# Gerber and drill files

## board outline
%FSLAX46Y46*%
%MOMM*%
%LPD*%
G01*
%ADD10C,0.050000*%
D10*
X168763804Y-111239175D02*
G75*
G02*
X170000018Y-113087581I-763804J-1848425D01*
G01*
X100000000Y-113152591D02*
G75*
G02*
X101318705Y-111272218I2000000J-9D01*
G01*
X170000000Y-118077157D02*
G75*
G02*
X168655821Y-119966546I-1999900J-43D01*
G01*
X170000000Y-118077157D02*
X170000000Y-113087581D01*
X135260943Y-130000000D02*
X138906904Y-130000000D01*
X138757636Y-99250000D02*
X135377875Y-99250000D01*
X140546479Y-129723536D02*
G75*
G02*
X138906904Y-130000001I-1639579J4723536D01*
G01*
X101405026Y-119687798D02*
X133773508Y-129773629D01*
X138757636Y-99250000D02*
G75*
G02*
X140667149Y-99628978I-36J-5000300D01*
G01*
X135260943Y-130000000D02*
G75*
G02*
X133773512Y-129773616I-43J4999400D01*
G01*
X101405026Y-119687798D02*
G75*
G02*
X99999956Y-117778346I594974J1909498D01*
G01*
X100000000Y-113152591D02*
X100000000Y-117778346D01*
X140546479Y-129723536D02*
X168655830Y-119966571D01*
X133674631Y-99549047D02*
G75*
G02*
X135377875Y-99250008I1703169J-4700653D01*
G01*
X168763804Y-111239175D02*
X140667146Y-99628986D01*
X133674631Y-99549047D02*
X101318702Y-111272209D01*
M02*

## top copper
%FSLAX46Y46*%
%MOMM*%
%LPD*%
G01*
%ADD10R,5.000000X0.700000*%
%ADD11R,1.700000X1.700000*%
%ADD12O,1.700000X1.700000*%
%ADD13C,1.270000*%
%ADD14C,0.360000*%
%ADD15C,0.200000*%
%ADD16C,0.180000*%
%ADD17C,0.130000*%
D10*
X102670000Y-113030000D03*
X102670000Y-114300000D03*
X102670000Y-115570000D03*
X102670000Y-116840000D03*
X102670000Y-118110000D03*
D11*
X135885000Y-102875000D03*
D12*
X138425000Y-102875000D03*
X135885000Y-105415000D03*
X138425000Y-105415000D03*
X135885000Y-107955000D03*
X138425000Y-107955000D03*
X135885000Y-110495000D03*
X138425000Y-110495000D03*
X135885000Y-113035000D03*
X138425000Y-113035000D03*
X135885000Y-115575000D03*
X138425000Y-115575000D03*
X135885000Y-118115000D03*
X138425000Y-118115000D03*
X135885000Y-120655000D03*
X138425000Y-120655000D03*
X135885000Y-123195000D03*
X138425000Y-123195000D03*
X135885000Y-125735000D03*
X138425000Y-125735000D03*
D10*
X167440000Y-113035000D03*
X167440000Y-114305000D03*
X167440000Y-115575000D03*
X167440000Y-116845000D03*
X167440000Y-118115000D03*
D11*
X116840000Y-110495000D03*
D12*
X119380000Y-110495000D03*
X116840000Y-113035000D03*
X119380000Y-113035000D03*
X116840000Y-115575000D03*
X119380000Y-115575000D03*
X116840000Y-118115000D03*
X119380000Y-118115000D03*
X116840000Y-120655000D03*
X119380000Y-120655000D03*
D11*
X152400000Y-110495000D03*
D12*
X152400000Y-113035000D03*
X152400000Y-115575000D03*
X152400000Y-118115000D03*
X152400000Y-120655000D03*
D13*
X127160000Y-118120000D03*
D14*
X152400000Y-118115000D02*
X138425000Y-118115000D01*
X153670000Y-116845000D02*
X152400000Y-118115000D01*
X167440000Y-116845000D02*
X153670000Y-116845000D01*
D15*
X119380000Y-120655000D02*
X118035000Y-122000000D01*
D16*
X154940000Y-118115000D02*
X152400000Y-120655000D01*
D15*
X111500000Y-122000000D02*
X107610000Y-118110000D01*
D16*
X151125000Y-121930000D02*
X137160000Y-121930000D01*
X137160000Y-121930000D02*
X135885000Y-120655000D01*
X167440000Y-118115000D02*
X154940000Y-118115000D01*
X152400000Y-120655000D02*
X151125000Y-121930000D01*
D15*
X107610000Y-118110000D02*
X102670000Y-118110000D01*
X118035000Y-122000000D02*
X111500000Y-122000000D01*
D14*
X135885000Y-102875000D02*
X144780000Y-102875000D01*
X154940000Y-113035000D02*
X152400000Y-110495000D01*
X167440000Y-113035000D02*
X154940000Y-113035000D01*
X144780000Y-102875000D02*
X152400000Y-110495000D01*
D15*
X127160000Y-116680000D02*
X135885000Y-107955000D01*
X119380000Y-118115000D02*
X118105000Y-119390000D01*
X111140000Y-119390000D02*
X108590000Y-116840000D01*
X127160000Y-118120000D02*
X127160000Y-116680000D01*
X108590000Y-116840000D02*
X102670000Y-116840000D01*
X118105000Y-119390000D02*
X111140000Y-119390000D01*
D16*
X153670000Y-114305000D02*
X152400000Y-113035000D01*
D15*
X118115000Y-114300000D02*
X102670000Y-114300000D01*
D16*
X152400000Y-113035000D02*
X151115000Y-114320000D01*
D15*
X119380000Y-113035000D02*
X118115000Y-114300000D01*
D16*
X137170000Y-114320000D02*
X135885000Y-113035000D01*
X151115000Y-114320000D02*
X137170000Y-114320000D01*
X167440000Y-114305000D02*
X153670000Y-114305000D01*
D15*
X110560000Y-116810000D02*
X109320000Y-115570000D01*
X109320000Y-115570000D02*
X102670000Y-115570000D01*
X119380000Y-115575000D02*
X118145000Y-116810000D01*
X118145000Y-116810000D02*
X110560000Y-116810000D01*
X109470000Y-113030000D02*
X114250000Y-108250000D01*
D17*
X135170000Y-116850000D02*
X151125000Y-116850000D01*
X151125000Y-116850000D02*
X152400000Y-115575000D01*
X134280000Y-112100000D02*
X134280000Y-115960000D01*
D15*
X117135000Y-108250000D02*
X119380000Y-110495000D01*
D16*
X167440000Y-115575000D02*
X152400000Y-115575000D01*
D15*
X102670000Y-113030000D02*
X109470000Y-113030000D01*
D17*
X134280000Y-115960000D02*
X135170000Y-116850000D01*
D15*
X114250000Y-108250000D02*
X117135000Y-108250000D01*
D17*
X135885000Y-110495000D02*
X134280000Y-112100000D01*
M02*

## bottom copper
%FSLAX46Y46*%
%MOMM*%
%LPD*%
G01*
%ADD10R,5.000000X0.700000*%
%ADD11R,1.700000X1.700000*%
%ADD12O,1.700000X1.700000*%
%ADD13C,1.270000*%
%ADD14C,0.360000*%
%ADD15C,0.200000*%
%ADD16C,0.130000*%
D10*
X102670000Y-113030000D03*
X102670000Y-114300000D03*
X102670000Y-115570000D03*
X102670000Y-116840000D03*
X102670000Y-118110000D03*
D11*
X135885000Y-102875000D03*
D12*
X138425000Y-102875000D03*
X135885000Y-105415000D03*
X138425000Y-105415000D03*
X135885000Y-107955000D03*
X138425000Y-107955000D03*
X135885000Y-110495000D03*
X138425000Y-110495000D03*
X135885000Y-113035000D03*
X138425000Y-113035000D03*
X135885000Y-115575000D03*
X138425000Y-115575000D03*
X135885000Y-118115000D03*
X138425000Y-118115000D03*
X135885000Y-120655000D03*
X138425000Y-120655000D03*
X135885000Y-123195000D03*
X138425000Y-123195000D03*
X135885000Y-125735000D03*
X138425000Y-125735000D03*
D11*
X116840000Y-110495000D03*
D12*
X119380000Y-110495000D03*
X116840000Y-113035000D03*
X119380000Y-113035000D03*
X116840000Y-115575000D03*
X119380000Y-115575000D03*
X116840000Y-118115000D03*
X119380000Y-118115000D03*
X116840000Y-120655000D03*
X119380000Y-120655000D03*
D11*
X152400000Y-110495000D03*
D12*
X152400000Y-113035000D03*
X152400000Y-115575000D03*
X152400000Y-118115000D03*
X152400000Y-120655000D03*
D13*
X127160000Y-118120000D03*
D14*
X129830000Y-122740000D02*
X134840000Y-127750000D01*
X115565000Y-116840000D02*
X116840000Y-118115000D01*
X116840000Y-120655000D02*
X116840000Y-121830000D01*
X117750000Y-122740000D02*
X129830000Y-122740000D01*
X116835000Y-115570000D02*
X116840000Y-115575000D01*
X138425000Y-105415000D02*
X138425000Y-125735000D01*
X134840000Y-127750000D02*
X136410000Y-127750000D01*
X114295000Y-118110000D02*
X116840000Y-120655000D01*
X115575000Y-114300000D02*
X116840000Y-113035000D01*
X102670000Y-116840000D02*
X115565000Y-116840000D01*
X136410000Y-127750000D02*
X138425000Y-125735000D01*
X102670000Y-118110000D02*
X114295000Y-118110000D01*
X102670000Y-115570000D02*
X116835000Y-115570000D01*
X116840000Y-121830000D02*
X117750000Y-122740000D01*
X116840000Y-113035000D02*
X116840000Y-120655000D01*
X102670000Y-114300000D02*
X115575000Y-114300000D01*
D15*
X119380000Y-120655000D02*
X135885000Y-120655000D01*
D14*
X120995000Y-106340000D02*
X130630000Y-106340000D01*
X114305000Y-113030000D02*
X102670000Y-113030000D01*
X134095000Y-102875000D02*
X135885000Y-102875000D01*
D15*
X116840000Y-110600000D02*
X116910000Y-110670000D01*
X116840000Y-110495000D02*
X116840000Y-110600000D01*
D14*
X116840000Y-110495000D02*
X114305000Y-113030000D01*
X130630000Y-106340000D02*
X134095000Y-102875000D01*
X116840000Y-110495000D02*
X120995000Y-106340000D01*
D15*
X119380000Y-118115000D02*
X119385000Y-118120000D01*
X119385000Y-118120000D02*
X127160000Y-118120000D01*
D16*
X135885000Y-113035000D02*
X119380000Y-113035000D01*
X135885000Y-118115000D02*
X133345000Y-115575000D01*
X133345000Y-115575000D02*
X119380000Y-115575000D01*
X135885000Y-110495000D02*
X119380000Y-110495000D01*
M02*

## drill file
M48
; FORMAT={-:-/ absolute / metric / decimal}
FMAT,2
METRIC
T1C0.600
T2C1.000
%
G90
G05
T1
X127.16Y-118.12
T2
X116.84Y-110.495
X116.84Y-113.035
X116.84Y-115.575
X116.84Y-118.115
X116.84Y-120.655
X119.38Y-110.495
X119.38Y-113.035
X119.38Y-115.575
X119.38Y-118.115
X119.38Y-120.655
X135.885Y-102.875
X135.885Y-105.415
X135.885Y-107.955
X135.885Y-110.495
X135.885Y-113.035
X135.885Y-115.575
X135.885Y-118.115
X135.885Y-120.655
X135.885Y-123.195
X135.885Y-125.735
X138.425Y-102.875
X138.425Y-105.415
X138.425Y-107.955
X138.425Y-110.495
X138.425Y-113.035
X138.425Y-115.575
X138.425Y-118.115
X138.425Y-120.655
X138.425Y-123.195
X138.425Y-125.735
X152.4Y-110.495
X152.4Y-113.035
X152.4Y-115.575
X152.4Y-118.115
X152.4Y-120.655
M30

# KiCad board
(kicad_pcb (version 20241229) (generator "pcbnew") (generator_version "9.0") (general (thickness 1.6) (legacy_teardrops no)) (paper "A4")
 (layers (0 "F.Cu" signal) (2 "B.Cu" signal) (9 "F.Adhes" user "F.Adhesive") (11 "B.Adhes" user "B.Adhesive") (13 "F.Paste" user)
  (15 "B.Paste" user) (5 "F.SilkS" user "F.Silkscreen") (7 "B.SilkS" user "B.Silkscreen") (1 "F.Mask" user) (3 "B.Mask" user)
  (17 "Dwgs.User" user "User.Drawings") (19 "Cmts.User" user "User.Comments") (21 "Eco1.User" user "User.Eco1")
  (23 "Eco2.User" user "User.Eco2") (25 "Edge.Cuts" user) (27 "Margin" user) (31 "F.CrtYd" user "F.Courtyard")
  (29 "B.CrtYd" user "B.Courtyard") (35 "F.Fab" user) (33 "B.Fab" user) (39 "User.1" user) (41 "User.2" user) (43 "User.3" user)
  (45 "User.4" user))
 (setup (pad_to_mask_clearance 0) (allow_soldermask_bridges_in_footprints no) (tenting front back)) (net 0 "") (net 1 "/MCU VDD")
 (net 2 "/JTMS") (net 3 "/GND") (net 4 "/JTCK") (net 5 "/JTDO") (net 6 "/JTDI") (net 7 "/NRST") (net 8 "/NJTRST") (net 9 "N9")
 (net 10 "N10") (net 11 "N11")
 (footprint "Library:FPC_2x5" (layer "F.Cu") (at 102.67 115.57 -90)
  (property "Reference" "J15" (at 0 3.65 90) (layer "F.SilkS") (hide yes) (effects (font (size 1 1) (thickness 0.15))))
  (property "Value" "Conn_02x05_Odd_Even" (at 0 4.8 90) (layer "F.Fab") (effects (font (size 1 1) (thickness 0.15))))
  (pad "1" smd rect (at -2.54 0 270) (size 0.7 5) (layers "B.Cu" "B.Mask" "B.Paste") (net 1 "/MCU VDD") (thermal_bridge_angle 45))
  (pad "2" smd rect (at -2.54 0 270) (size 0.7 5) (layers "F.Cu" "F.Mask" "F.Paste") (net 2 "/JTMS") (thermal_bridge_angle 45))
  (pad "3" smd rect (at -1.27 0 270) (size 0.7 5) (layers "B.Cu" "B.Mask" "B.Paste") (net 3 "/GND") (thermal_bridge_angle 45))
  (pad "4" smd rect (at -1.27 0 270) (size 0.7 5) (layers "F.Cu" "F.Mask" "F.Paste") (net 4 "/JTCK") (thermal_bridge_angle 45))
  (pad "5" smd rect (at 0 0 270) (size 0.7 5) (layers "B.Cu" "B.Mask" "B.Paste") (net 3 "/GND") (thermal_bridge_angle 45))
  (pad "6" smd rect (at 0 0 270) (size 0.7 5) (layers "F.Cu" "F.Mask" "F.Paste") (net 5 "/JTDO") (thermal_bridge_angle 45))
  (pad "7" smd rect (at 1.27 0 270) (size 0.7 5) (layers "B.Cu" "B.Mask" "B.Paste") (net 3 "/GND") (thermal_bridge_angle 45))
  (pad "8" smd rect (at 1.27 0 270) (size 0.7 5) (layers "F.Cu" "F.Mask" "F.Paste") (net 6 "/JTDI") (thermal_bridge_angle 45))
  (pad "9" smd rect (at 2.54 0 270) (size 0.7 5) (layers "B.Cu" "B.Mask" "B.Paste") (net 3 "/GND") (thermal_bridge_angle 45))
  (pad "10" smd rect (at 2.54 0 270) (size 0.7 5) (layers "F.Cu" "F.Mask" "F.Paste") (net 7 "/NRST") (thermal_bridge_angle 45)))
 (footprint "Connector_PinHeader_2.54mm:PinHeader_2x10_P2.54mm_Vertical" (layer "F.Cu") (at 135.885 102.875)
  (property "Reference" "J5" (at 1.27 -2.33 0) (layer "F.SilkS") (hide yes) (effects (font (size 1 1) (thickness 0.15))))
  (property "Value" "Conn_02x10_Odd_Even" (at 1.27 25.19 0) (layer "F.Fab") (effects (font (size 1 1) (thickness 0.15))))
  (pad "1" thru_hole rect (at 0 0) (size 1.7 1.7) (drill 1) (layers "*.Cu" "*.Mask") (remove_unused_layers no) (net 1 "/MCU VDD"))
  (pad "2" thru_hole oval (at 2.54 0) (size 1.7 1.7) (drill 1) (layers "*.Cu" "*.Mask") (remove_unused_layers no) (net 1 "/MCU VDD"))
  (pad "3" thru_hole oval (at 0 2.54) (size 1.7 1.7) (drill 1) (layers "*.Cu" "*.Mask") (remove_unused_layers no) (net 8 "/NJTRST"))
  (pad "4" thru_hole oval (at 2.54 2.54) (size 1.7 1.7) (drill 1) (layers "*.Cu" "*.Mask") (remove_unused_layers no) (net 3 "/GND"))
  (pad "5" thru_hole oval (at 0 5.08) (size 1.7 1.7) (drill 1) (layers "*.Cu" "*.Mask") (remove_unused_layers no) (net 6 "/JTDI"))
  (pad "6" thru_hole oval (at 2.54 5.08) (size 1.7 1.7) (drill 1) (layers "*.Cu" "*.Mask") (remove_unused_layers no) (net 3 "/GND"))
  (pad "7" thru_hole oval (at 0 7.62) (size 1.7 1.7) (drill 1) (layers "*.Cu" "*.Mask") (remove_unused_layers no) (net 2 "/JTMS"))
  (pad "8" thru_hole oval (at 2.54 7.62) (size 1.7 1.7) (drill 1) (layers "*.Cu" "*.Mask") (remove_unused_layers no) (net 3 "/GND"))
  (pad "9" thru_hole oval (at 0 10.16) (size 1.7 1.7) (drill 1) (layers "*.Cu" "*.Mask") (remove_unused_layers no) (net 4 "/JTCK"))
  (pad "10" thru_hole oval (at 2.54 10.16) (size 1.7 1.7) (drill 1) (layers "*.Cu" "*.Mask") (remove_unused_layers no) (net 3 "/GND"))
  (pad "11" thru_hole oval (at 0 12.7) (size 1.7 1.7) (drill 1) (layers "*.Cu" "*.Mask") (remove_unused_layers no) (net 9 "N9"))
  (pad "12" thru_hole oval (at 2.54 12.7) (size 1.7 1.7) (drill 1) (layers "*.Cu" "*.Mask") (remove_unused_layers no) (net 3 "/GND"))
  (pad "13" thru_hole oval (at 0 15.24) (size 1.7 1.7) (drill 1) (layers "*.Cu" "*.Mask") (remove_unused_layers no) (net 5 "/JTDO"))
  (pad "14" thru_hole oval (at 2.54 15.24) (size 1.7 1.7) (drill 1) (layers "*.Cu" "*.Mask") (remove_unused_layers no) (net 3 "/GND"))
  (pad "15" thru_hole oval (at 0 17.78) (size 1.7 1.7) (drill 1) (layers "*.Cu" "*.Mask") (remove_unused_layers no) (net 7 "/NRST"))
  (pad "16" thru_hole oval (at 2.54 17.78) (size 1.7 1.7) (drill 1) (layers "*.Cu" "*.Mask") (remove_unused_layers no) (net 3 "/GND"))
  (pad "17" thru_hole oval (at 0 20.32) (size 1.7 1.7) (drill 1) (layers "*.Cu" "*.Mask") (remove_unused_layers no) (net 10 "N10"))
  (pad "18" thru_hole oval (at 2.54 20.32) (size 1.7 1.7) (drill 1) (layers "*.Cu" "*.Mask") (remove_unused_layers no) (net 3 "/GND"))
  (pad "19" thru_hole oval (at 0 22.86) (size 1.7 1.7) (drill 1) (layers "*.Cu" "*.Mask") (remove_unused_layers no) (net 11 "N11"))
  (pad "20" thru_hole oval (at 2.54 22.86) (size 1.7 1.7) (drill 1) (layers "*.Cu" "*.Mask") (remove_unused_layers no) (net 3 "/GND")))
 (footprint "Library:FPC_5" (layer "F.Cu") (at 167.44 115.575 -90)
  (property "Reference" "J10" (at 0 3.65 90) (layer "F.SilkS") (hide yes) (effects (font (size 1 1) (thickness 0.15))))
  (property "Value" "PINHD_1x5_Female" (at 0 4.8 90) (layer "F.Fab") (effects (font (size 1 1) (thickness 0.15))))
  (pad "1" smd rect (at -2.54 0 270) (size 0.7 5) (layers "F.Cu" "F.Mask" "F.Paste") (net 1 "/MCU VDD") (thermal_bridge_angle 45))
  (pad "2" smd rect (at -1.27 0 270) (size 0.7 5) (layers "F.Cu" "F.Mask" "F.Paste") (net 4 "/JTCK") (thermal_bridge_angle 45))
  (pad "3" smd rect (at 0 0 270) (size 0.7 5) (layers "F.Cu" "F.Mask" "F.Paste") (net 2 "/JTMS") (thermal_bridge_angle 45))
  (pad "4" smd rect (at 1.27 0 270) (size 0.7 5) (layers "F.Cu" "F.Mask" "F.Paste") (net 3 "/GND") (thermal_bridge_angle 45))
  (pad "5" smd rect (at 2.54 0 270) (size 0.7 5) (layers "F.Cu" "F.Mask" "F.Paste") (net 7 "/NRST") (thermal_bridge_angle 45)))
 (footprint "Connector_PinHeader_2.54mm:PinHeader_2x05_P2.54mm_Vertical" (layer "F.Cu") (at 116.84 110.495)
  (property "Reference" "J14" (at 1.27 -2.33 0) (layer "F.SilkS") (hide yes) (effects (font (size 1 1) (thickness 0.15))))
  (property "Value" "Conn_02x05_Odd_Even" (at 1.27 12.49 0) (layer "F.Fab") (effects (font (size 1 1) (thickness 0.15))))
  (pad "1" thru_hole rect (at 0 0) (size 1.7 1.7) (drill 1) (layers "*.Cu" "*.Mask") (remove_unused_layers no) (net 1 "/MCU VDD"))
  (pad "2" thru_hole oval (at 2.54 0) (size 1.7 1.7) (drill 1) (layers "*.Cu" "*.Mask") (remove_unused_layers no) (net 2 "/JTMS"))
  (pad "3" thru_hole oval (at 0 2.54) (size 1.7 1.7) (drill 1) (layers "*.Cu" "*.Mask") (remove_unused_layers no) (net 3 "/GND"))
  (pad "4" thru_hole oval (at 2.54 2.54) (size 1.7 1.7) (drill 1) (layers "*.Cu" "*.Mask") (remove_unused_layers no) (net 4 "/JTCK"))
  (pad "5" thru_hole oval (at 0 5.08) (size 1.7 1.7) (drill 1) (layers "*.Cu" "*.Mask") (remove_unused_layers no) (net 3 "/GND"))
  (pad "6" thru_hole oval (at 2.54 5.08) (size 1.7 1.7) (drill 1) (layers "*.Cu" "*.Mask") (remove_unused_layers no) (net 5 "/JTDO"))
  (pad "7" thru_hole oval (at 0 7.62) (size 1.7 1.7) (drill 1) (layers "*.Cu" "*.Mask") (remove_unused_layers no) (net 3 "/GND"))
  (pad "8" thru_hole oval (at 2.54 7.62) (size 1.7 1.7) (drill 1) (layers "*.Cu" "*.Mask") (remove_unused_layers no) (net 6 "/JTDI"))
  (pad "9" thru_hole oval (at 0 10.16) (size 1.7 1.7) (drill 1) (layers "*.Cu" "*.Mask") (remove_unused_layers no) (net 3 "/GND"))
  (pad "10" thru_hole oval (at 2.54 10.16) (size 1.7 1.7) (drill 1) (layers "*.Cu" "*.Mask") (remove_unused_layers no) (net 7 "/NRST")))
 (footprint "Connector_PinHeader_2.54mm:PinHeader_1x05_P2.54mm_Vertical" (layer "F.Cu") (at 152.4 110.495)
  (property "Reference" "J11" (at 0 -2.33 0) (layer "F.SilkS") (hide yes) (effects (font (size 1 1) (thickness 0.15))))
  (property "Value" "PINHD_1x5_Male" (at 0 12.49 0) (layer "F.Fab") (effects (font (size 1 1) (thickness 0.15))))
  (pad "1" thru_hole rect (at 0 0) (size 1.7 1.7) (drill 1) (layers "*.Cu" "*.Mask") (remove_unused_layers no) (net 1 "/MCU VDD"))
  (pad "2" thru_hole oval (at 0 2.54) (size 1.7 1.7) (drill 1) (layers "*.Cu" "*.Mask") (remove_unused_layers no) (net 4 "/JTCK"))
  (pad "3" thru_hole oval (at 0 5.08) (size 1.7 1.7) (drill 1) (layers "*.Cu" "*.Mask") (remove_unused_layers no) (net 2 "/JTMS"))
  (pad "4" thru_hole oval (at 0 7.62) (size 1.7 1.7) (drill 1) (layers "*.Cu" "*.Mask") (remove_unused_layers no) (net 3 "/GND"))
  (pad "5" thru_hole oval (at 0 10.16) (size 1.7 1.7) (drill 1) (layers "*.Cu" "*.Mask") (remove_unused_layers no) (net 7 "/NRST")))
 (gr_arc (start 168.763804 111.239175) (mid 169.662469 111.975737) (end 170 113.087581) (stroke (width 0.05) (type default))
  (layer "Edge.Cuts"))
 (gr_arc (start 100 113.152591) (mid 100.362537 112.004247) (end 101.318702 111.272209) (stroke (width 0.05) (type default))
  (layer "Edge.Cuts"))
 (gr_arc (start 170 118.077157) (mid 169.629688 119.23656) (end 168.65583 119.966571) (stroke (width 0.05) (type default))
  (layer "Edge.Cuts"))
 (gr_line (start 170 118.077157) (end 170 113.087581) (stroke (width 0.05) (type default)) (layer "Edge.Cuts"))
 (gr_line (start 135.260943 130) (end 138.906904 130) (stroke (width 0.05) (type default)) (layer "Edge.Cuts"))
 (gr_line (start 138.757636 99.25) (end 135.377875 99.25) (stroke (width 0.05) (type default)) (layer "Edge.Cuts"))
 (gr_arc (start 140.546479 129.723536) (mid 139.738264 129.930399) (end 138.906904 130) (stroke (width 0.05) (type default))
  (layer "Edge.Cuts"))
 (gr_line (start 101.405026 119.687798) (end 133.773508 129.773629) (stroke (width 0.05) (type default)) (layer "Edge.Cuts"))
 (gr_arc (start 138.757636 99.25) (mid 139.731012 99.345668) (end 140.667146 99.628986) (stroke (width 0.05) (type default))
  (layer "Edge.Cuts"))
 (gr_arc (start 135.260943 130) (mid 134.508661 129.94309) (end 133.773508 129.773629) (stroke (width 0.05) (type default))
  (layer "Edge.Cuts"))
 (gr_arc (start 101.405026 119.687798) (mid 100.389108 118.963684) (end 100 117.778346) (stroke (width 0.05) (type default))
  (layer "Edge.Cuts"))
 (gr_line (start 100 113.152591) (end 100 117.778346) (stroke (width 0.05) (type default)) (layer "Edge.Cuts"))
 (gr_line (start 140.546479 129.723536) (end 168.65583 119.966571) (stroke (width 0.05) (type default)) (layer "Edge.Cuts"))
 (gr_arc (start 133.674631 99.549047) (mid 134.513226 99.325325) (end 135.377875 99.25) (stroke (width 0.05) (type default))
  (layer "Edge.Cuts"))
 (gr_line (start 168.763804 111.239175) (end 140.667146 99.628986) (stroke (width 0.05) (type default)) (layer "Edge.Cuts"))
 (gr_line (start 133.674631 99.549047) (end 101.318702 111.272209) (stroke (width 0.05) (type default)) (layer "Edge.Cuts"))
 (segment (start 152.4 118.115) (end 138.425 118.115) (width 0.36) (layer "F.Cu") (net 3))
 (segment (start 153.67 116.845) (end 152.4 118.115) (width 0.36) (layer "F.Cu") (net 3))
 (segment (start 167.44 116.845) (end 153.67 116.845) (width 0.36) (layer "F.Cu") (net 3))
 (segment (start 129.83 122.74) (end 134.84 127.75) (width 0.36) (layer "B.Cu") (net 3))
 (segment (start 115.565 116.84) (end 116.84 118.115) (width 0.36) (layer "B.Cu") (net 3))
 (segment (start 116.84 120.655) (end 116.84 121.83) (width 0.36) (layer "B.Cu") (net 3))
 (segment (start 117.75 122.74) (end 129.83 122.74) (width 0.36) (layer "B.Cu") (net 3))
 (segment (start 116.835 115.57) (end 116.84 115.575) (width 0.36) (layer "B.Cu") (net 3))
 (segment (start 138.425 105.415) (end 138.425 125.735) (width 0.36) (layer "B.Cu") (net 3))
 (segment (start 134.84 127.75) (end 136.41 127.75) (width 0.36) (layer "B.Cu") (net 3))
 (segment (start 114.295 118.11) (end 116.84 120.655) (width 0.36) (layer "B.Cu") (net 3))
 (segment (start 115.575 114.3) (end 116.84 113.035) (width 0.36) (layer "B.Cu") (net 3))
 (segment (start 102.67 116.84) (end 115.565 116.84) (width 0.36) (layer "B.Cu") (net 3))
 (segment (start 136.41 127.75) (end 138.425 125.735) (width 0.36) (layer "B.Cu") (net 3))
 (segment (start 102.67 118.11) (end 114.295 118.11) (width 0.36) (layer "B.Cu") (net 3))
 (segment (start 102.67 115.57) (end 116.835 115.57) (width 0.36) (layer "B.Cu") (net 3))
 (segment (start 116.84 121.83) (end 117.75 122.74) (width 0.36) (layer "B.Cu") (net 3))
 (segment (start 116.84 113.035) (end 116.84 120.655) (width 0.36) (layer "B.Cu") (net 3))
 (segment (start 102.67 114.3) (end 115.575 114.3) (width 0.36) (layer "B.Cu") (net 3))
 (segment (start 119.38 120.655) (end 118.035 122) (width 0.2) (layer "F.Cu") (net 7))
 (segment (start 154.94 118.115) (end 152.4 120.655) (width 0.18) (layer "F.Cu") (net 7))
 (segment (start 111.5 122) (end 107.61 118.11) (width 0.2) (layer "F.Cu") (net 7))
 (segment (start 151.125 121.93) (end 137.16 121.93) (width 0.18) (layer "F.Cu") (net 7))
 (segment (start 137.16 121.93) (end 135.885 120.655) (width 0.18) (layer "F.Cu") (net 7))
 (segment (start 167.44 118.115) (end 154.94 118.115) (width 0.18) (layer "F.Cu") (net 7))
 (segment (start 152.4 120.655) (end 151.125 121.93) (width 0.18) (layer "F.Cu") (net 7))
 (segment (start 107.61 118.11) (end 102.67 118.11) (width 0.2) (layer "F.Cu") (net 7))
 (segment (start 118.035 122) (end 111.5 122) (width 0.2) (layer "F.Cu") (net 7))
 (segment (start 119.38 120.655) (end 135.885 120.655) (width 0.2) (layer "B.Cu") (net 7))
 (segment (start 135.885 102.875) (end 144.78 102.875) (width 0.36) (layer "F.Cu") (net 1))
 (segment (start 154.94 113.035) (end 152.4 110.495) (width 0.36) (layer "F.Cu") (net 1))
 (segment (start 167.44 113.035) (end 154.94 113.035) (width 0.36) (layer "F.Cu") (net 1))
 (segment (start 144.78 102.875) (end 152.4 110.495) (width 0.36) (layer "F.Cu") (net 1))
 (segment (start 120.995 106.34) (end 130.63 106.34) (width 0.36) (layer "B.Cu") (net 1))
 (segment (start 114.305 113.03) (end 102.67 113.03) (width 0.36) (layer "B.Cu") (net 1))
 (segment (start 134.095 102.875) (end 135.885 102.875) (width 0.36) (layer "B.Cu") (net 1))
 (segment (start 116.84 110.6) (end 116.91 110.67) (width 0.2) (layer "B.Cu") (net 1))
 (segment (start 116.84 110.495) (end 116.84 110.6) (width 0.2) (layer "B.Cu") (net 1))
 (segment (start 116.84 110.495) (end 114.305 113.03) (width 0.36) (layer "B.Cu") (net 1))
 (segment (start 130.63 106.34) (end 134.095 102.875) (width 0.36) (layer "B.Cu") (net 1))
 (segment (start 116.84 110.495) (end 120.995 106.34) (width 0.36) (layer "B.Cu") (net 1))
 (segment (start 127.16 116.68) (end 135.885 107.955) (width 0.2) (layer "F.Cu") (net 6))
 (segment (start 119.38 118.115) (end 118.105 119.39) (width 0.2) (layer "F.Cu") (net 6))
 (segment (start 111.14 119.39) (end 108.59 116.84) (width 0.2) (layer "F.Cu") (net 6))
 (segment (start 127.16 118.12) (end 127.16 116.68) (width 0.2) (layer "F.Cu") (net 6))
 (segment (start 108.59 116.84) (end 102.67 116.84) (width 0.2) (layer "F.Cu") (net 6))
 (segment (start 118.105 119.39) (end 111.14 119.39) (width 0.2) (layer "F.Cu") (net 6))
 (via (at 127.16 118.12) (size 1.27) (drill 0.6) (layers "F.Cu" "B.Cu") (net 6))
 (segment (start 119.38 118.115) (end 119.385 118.12) (width 0.2) (layer "B.Cu") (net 6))
 (segment (start 119.385 118.12) (end 127.16 118.12) (width 0.2) (layer "B.Cu") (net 6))
 (segment (start 153.67 114.305) (end 152.4 113.035) (width 0.18) (layer "F.Cu") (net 4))
 (segment (start 118.115 114.3) (end 102.67 114.3) (width 0.2) (layer "F.Cu") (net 4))
 (segment (start 152.4 113.035) (end 151.115 114.32) (width 0.18) (layer "F.Cu") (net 4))
 (segment (start 119.38 113.035) (end 118.115 114.3) (width 0.2) (layer "F.Cu") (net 4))
 (segment (start 137.17 114.32) (end 135.885 113.035) (width 0.18) (layer "F.Cu") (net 4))
 (segment (start 151.115 114.32) (end 137.17 114.32) (width 0.18) (layer "F.Cu") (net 4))
 (segment (start 167.44 114.305) (end 153.67 114.305) (width 0.18) (layer "F.Cu") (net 4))
 (segment (start 135.885 113.035) (end 119.38 113.035) (width 0.13) (layer "B.Cu") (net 4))
 (segment (start 110.56 116.81) (end 109.32 115.57) (width 0.2) (layer "F.Cu") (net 5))
 (segment (start 109.32 115.57) (end 102.67 115.57) (width 0.2) (layer "F.Cu") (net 5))
 (segment (start 119.38 115.575) (end 118.145 116.81) (width 0.2) (layer "F.Cu") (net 5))
 (segment (start 118.145 116.81) (end 110.56 116.81) (width 0.2) (layer "F.Cu") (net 5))
 (segment (start 135.885 118.115) (end 133.345 115.575) (width 0.13) (layer "B.Cu") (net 5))
 (segment (start 133.345 115.575) (end 119.38 115.575) (width 0.13) (layer "B.Cu") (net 5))
 (segment (start 109.47 113.03) (end 114.25 108.25) (width 0.2) (layer "F.Cu") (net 2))
 (segment (start 135.17 116.85) (end 151.125 116.85) (width 0.13) (layer "F.Cu") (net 2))
 (segment (start 151.125 116.85) (end 152.4 115.575) (width 0.13) (layer "F.Cu") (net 2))
 (segment (start 134.28 112.1) (end 134.28 115.96) (width 0.13) (layer "F.Cu") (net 2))
 (segment (start 117.135 108.25) (end 119.38 110.495) (width 0.2) (layer "F.Cu") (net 2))
 (segment (start 167.44 115.575) (end 152.4 115.575) (width 0.18) (layer "F.Cu") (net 2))
 (segment (start 102.67 113.03) (end 109.47 113.03) (width 0.2) (layer "F.Cu") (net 2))
 (segment (start 134.28 115.96) (end 135.17 116.85) (width 0.13) (layer "F.Cu") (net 2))
 (segment (start 114.25 108.25) (end 117.135 108.25) (width 0.2) (layer "F.Cu") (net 2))
 (segment (start 135.885 110.495) (end 134.28 112.1) (width 0.13) (layer "F.Cu") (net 2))
 (segment (start 135.885 110.495) (end 119.38 110.495) (width 0.13) (layer "B.Cu") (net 2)))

